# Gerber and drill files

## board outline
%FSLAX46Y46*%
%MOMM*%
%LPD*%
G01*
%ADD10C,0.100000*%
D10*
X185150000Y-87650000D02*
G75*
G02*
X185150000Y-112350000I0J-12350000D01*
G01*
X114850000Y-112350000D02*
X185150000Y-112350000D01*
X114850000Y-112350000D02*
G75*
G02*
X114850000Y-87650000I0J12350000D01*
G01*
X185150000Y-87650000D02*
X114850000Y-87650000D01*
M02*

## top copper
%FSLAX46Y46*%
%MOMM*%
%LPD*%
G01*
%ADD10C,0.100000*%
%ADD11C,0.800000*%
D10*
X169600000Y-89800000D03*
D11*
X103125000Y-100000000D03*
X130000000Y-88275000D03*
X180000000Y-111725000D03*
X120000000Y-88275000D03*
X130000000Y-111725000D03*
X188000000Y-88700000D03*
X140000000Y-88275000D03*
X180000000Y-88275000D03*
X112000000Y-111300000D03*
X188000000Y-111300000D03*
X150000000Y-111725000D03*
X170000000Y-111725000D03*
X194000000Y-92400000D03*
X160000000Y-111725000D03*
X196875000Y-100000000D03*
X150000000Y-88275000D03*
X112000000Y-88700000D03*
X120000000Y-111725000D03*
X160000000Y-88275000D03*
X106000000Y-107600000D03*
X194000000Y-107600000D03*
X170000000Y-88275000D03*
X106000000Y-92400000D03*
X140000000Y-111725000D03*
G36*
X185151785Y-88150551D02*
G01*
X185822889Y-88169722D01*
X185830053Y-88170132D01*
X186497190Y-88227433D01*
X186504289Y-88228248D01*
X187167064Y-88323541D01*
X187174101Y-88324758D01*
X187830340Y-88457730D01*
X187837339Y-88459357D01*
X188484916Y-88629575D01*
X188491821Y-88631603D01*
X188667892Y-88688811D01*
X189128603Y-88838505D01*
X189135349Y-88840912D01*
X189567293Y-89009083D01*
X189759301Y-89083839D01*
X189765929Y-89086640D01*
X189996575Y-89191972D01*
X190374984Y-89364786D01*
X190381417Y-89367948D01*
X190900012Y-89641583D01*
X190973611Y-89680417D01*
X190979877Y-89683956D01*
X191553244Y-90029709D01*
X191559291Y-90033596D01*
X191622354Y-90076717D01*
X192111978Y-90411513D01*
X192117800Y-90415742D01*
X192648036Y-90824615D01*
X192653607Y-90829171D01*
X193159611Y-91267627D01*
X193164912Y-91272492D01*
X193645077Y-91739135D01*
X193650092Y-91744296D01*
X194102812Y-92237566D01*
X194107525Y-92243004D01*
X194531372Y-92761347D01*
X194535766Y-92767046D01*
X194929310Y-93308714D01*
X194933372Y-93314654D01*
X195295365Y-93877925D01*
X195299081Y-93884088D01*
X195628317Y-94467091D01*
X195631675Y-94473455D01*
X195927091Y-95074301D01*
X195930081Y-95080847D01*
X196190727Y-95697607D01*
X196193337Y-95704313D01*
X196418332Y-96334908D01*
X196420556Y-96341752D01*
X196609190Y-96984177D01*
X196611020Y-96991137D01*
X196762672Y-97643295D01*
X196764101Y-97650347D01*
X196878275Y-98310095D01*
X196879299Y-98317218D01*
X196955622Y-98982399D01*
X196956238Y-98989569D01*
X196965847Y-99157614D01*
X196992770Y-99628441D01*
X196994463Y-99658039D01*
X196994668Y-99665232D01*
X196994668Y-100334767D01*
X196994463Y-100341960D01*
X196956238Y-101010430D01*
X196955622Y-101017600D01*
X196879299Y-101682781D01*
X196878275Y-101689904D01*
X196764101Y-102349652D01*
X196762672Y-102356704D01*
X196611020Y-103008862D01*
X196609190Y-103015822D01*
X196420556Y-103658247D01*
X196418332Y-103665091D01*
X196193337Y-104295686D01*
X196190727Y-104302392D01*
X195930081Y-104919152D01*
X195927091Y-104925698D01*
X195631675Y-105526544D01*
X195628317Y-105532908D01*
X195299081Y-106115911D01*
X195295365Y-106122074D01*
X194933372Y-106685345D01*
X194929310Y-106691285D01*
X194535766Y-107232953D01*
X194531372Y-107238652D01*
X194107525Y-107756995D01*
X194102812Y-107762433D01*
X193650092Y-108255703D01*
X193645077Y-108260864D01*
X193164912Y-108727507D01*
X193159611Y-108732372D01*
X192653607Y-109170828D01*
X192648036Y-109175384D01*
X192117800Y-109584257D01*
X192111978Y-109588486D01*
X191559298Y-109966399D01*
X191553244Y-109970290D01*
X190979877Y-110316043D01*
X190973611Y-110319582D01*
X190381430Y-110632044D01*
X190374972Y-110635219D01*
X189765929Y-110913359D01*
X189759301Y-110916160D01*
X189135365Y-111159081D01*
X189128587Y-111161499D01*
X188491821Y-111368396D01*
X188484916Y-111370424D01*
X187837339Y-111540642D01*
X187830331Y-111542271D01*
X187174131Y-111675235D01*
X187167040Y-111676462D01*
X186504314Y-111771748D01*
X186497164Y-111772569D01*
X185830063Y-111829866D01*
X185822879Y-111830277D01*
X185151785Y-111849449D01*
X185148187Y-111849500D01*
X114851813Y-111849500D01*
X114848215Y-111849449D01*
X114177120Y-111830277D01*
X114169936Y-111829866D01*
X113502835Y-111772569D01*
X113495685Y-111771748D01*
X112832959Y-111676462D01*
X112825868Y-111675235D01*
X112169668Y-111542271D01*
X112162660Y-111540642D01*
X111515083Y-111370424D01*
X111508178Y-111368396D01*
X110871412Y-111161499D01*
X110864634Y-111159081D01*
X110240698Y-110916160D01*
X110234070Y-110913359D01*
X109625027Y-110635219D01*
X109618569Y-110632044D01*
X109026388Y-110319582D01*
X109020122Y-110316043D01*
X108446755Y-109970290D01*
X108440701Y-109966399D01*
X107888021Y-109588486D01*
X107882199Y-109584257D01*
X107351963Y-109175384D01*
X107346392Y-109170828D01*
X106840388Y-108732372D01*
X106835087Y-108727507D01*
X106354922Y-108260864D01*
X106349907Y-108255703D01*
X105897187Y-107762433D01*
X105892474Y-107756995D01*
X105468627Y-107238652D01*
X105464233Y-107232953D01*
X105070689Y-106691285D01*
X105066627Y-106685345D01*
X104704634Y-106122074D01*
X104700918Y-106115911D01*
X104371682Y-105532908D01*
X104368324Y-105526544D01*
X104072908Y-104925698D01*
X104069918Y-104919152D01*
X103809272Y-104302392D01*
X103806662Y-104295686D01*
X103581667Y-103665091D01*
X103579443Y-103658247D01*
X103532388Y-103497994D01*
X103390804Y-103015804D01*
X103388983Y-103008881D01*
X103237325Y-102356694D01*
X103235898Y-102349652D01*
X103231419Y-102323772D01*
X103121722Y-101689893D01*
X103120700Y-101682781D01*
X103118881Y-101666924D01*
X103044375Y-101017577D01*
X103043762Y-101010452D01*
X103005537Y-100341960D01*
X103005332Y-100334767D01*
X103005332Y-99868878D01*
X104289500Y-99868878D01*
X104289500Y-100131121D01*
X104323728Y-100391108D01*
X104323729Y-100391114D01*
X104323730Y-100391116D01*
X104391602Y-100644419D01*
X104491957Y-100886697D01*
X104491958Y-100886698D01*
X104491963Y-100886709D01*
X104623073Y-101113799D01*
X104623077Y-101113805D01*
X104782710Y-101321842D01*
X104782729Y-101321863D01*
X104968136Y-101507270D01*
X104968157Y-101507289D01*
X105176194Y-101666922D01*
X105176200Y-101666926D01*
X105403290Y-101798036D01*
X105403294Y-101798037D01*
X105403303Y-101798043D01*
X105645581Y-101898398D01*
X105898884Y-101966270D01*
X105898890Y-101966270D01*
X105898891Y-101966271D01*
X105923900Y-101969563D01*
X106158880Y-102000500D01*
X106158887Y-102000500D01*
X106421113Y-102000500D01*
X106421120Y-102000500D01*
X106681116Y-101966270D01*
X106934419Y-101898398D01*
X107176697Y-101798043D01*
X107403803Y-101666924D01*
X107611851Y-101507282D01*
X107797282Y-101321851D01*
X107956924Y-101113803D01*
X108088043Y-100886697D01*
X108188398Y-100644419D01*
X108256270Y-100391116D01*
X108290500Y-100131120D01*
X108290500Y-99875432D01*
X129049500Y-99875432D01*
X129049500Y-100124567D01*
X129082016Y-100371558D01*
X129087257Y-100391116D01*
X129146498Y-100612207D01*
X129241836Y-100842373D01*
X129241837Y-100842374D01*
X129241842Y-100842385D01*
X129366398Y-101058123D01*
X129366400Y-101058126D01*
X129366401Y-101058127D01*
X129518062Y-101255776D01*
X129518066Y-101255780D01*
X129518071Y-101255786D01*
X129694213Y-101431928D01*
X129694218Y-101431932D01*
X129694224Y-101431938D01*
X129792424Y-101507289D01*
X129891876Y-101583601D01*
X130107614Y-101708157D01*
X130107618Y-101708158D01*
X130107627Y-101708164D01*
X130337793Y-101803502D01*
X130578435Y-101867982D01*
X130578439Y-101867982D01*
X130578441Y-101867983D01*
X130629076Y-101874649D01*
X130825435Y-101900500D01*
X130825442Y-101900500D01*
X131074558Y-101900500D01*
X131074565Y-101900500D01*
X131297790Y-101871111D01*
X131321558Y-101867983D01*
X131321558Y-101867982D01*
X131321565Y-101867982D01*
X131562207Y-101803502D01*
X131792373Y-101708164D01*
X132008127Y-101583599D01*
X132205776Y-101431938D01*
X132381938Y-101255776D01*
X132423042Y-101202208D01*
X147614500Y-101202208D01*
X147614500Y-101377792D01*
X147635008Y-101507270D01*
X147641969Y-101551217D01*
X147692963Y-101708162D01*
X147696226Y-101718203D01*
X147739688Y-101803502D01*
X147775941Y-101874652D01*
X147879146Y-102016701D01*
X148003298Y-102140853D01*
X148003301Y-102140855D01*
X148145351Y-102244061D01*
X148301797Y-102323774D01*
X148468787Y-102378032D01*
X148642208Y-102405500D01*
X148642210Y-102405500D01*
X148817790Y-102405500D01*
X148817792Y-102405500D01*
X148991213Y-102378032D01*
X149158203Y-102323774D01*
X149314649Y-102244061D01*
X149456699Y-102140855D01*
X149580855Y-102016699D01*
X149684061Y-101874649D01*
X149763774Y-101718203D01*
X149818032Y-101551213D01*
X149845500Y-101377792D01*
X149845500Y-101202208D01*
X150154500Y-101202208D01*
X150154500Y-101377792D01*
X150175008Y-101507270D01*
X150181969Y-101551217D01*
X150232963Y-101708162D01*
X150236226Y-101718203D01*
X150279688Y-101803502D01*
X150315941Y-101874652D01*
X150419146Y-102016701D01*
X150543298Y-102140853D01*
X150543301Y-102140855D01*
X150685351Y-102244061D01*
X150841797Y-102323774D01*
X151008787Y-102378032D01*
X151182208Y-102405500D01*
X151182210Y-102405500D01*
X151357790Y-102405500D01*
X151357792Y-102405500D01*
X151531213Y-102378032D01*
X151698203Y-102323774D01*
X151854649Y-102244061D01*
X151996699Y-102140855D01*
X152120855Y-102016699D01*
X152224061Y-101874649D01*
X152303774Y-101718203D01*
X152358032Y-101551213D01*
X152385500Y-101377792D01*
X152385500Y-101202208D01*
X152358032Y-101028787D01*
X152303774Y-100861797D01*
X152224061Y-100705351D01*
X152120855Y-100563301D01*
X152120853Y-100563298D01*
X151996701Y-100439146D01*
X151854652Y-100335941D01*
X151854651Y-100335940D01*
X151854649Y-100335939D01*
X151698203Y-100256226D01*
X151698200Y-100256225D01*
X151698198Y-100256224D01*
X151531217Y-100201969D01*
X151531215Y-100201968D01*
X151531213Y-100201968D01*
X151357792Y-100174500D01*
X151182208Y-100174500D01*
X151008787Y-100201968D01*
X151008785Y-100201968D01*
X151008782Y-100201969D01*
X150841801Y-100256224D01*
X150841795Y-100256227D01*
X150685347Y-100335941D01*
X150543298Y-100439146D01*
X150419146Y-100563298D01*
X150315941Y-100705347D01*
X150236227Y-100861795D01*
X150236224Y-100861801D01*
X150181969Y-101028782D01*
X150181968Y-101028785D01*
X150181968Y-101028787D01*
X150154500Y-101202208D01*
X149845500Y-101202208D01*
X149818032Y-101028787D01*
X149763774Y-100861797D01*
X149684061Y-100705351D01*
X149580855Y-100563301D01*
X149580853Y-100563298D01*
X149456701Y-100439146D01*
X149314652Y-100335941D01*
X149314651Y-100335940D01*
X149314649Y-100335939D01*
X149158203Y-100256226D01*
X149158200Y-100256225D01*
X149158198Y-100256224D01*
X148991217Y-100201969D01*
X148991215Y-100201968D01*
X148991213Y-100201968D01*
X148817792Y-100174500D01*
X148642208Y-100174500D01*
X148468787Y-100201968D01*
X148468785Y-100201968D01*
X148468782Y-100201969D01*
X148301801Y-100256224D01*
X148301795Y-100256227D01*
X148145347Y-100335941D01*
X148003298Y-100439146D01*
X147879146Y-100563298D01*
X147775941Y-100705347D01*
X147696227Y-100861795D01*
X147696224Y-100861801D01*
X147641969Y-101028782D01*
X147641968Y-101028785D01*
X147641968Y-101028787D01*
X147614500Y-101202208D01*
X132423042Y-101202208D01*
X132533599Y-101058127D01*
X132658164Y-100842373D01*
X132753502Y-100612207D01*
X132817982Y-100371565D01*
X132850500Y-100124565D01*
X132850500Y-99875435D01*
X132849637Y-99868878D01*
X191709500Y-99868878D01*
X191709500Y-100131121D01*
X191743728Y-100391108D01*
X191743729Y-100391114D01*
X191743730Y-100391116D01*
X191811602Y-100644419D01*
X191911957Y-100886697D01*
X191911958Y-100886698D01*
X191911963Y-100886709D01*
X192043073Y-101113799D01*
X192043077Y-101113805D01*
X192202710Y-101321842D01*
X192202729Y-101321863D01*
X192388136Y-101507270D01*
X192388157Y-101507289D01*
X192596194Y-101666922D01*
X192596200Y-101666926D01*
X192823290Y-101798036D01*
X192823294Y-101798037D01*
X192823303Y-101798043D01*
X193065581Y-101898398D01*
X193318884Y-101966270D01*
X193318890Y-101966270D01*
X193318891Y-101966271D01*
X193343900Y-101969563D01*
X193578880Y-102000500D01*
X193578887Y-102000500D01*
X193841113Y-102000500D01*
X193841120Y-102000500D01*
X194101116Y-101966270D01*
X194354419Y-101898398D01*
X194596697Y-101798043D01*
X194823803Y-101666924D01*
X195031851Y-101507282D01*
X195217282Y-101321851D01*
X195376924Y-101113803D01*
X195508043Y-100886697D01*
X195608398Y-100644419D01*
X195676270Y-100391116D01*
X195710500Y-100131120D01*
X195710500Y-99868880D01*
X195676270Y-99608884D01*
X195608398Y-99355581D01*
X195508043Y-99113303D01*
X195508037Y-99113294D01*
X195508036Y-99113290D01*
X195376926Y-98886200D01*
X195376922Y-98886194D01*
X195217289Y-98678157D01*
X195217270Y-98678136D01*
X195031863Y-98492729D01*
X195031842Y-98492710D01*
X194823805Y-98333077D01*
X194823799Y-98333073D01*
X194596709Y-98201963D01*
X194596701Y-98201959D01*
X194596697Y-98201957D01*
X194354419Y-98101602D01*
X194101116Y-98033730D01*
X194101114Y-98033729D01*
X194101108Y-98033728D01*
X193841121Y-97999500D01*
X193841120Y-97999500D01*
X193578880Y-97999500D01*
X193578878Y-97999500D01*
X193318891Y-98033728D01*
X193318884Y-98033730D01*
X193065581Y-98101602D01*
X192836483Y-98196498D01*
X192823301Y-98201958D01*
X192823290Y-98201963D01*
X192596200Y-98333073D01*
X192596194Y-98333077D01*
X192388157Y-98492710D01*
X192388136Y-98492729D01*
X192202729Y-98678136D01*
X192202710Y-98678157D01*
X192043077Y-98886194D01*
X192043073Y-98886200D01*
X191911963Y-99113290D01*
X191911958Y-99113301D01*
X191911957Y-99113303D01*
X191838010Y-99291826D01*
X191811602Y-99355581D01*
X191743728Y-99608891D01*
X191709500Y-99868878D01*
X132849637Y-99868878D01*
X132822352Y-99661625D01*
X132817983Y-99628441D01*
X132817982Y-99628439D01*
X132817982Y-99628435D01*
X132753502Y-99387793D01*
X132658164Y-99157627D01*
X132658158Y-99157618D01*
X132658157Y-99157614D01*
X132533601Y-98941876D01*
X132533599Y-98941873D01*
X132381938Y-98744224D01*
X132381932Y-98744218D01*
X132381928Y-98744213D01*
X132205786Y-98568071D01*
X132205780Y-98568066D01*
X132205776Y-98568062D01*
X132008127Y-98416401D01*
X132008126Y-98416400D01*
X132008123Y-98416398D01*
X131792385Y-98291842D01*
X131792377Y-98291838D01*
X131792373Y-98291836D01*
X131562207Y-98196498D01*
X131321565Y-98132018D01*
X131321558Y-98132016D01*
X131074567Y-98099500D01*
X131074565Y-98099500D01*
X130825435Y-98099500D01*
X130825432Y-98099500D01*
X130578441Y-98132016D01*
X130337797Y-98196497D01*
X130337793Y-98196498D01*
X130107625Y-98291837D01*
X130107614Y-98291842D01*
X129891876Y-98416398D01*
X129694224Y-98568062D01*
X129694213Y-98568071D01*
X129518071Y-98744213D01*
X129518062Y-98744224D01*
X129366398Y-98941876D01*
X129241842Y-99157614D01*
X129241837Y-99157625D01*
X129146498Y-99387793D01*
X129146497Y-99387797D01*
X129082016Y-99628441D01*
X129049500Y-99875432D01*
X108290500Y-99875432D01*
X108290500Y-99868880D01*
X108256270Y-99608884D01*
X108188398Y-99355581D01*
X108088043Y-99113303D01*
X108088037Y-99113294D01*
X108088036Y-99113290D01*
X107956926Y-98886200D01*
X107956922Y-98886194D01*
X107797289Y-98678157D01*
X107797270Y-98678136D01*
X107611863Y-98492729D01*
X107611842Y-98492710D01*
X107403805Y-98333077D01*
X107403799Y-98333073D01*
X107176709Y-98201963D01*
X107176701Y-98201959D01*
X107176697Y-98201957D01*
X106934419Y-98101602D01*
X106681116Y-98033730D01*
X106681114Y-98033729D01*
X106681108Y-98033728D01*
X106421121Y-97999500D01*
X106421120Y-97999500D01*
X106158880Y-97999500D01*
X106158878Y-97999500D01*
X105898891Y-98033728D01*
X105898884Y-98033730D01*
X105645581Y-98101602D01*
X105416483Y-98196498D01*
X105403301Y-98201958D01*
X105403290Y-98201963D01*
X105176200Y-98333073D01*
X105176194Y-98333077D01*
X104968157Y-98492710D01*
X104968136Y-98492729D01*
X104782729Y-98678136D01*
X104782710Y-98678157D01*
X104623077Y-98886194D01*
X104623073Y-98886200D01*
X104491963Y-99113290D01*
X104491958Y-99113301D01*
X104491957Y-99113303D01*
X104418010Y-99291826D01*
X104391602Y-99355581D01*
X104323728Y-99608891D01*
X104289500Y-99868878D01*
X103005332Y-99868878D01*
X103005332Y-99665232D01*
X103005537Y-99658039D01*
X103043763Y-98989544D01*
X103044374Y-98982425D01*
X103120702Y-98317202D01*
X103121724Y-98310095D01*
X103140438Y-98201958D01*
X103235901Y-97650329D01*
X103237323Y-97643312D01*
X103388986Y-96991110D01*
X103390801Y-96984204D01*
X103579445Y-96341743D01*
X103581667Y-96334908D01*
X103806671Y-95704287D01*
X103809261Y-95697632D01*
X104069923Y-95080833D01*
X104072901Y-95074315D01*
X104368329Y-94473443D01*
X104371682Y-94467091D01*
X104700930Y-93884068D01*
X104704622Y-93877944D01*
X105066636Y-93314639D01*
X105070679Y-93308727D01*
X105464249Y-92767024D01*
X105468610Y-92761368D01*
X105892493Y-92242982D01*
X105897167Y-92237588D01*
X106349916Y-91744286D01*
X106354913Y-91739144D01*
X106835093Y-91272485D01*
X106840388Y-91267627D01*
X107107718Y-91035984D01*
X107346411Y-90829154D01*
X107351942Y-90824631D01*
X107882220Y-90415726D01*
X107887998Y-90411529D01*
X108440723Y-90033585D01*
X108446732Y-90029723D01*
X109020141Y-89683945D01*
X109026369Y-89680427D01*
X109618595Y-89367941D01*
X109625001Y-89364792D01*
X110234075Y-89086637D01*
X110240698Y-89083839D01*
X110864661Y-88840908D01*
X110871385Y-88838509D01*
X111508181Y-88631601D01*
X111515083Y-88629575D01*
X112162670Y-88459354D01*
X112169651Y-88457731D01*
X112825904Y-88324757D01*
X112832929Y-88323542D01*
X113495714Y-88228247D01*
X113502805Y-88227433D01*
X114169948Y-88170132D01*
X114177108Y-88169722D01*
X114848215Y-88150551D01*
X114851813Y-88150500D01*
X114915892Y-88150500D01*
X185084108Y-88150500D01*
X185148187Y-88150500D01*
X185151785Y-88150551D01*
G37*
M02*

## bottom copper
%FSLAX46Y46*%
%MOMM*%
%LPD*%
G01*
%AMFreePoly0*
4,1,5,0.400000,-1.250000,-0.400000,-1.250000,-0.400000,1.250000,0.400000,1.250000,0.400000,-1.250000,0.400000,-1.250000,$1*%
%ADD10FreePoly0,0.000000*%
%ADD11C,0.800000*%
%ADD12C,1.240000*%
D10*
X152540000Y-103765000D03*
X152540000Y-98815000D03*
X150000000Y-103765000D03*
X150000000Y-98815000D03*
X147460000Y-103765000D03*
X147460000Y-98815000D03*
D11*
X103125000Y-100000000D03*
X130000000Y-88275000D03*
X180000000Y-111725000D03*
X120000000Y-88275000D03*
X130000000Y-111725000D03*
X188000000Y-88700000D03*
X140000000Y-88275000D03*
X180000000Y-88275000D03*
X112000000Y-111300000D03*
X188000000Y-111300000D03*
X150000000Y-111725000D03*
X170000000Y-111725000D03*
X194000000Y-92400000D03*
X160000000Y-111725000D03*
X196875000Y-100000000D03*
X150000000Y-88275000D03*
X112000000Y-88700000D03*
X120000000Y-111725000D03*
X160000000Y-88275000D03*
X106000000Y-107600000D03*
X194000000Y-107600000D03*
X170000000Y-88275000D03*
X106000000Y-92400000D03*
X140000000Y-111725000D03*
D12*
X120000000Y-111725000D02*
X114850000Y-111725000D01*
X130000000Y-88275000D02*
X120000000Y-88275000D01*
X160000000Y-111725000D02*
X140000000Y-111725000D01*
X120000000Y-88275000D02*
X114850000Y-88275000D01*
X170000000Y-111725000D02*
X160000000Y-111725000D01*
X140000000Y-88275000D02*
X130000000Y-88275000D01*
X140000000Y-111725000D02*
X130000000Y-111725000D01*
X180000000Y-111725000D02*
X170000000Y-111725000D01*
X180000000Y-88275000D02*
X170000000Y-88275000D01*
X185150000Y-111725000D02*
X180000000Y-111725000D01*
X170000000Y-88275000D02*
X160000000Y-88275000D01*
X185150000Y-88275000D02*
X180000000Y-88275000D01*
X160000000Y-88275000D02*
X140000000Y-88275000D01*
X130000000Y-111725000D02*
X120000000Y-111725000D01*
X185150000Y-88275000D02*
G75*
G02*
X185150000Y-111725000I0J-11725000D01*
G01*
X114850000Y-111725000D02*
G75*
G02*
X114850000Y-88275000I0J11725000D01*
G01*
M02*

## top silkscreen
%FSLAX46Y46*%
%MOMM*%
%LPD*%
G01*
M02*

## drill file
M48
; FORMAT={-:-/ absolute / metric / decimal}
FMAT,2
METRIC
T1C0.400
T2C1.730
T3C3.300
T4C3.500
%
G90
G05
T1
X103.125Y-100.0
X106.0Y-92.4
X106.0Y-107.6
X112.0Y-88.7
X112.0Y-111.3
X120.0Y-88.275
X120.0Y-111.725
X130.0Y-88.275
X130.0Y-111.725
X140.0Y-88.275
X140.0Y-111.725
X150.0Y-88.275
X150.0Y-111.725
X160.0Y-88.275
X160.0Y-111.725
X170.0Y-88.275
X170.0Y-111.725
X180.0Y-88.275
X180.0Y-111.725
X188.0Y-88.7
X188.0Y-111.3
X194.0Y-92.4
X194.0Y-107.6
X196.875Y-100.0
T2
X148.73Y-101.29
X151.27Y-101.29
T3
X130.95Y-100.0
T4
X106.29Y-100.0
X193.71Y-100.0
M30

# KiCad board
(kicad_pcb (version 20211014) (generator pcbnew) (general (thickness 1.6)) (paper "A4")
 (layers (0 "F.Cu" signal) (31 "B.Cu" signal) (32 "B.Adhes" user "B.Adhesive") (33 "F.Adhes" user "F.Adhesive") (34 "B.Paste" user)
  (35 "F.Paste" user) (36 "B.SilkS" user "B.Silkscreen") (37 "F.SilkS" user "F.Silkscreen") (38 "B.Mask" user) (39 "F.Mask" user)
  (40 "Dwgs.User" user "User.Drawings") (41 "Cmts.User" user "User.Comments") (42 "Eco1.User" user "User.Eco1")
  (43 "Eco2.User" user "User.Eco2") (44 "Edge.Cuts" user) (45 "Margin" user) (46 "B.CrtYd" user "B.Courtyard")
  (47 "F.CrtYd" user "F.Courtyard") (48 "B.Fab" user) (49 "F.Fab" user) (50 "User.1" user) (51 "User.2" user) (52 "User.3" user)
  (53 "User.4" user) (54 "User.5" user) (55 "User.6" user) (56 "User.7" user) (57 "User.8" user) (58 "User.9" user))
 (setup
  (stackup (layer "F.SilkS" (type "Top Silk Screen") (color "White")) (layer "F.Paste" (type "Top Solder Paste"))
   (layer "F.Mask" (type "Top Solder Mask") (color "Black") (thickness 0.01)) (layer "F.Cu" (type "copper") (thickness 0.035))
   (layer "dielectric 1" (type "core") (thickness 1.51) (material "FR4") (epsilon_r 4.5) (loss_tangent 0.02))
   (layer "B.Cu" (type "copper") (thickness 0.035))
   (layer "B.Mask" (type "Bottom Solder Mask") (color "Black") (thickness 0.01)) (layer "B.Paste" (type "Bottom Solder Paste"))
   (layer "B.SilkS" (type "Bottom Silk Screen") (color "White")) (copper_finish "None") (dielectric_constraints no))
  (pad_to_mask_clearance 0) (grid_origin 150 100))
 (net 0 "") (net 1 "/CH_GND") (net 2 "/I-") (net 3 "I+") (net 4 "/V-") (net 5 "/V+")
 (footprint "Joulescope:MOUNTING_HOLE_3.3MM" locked (layer "F.Cu") (at 130.95 100)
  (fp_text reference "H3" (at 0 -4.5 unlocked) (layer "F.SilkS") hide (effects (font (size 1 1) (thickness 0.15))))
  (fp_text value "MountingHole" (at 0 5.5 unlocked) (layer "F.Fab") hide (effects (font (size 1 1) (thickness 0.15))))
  (pad "" np_thru_hole circle locked (at 0 0) (size 3.3 3.3) (drill 3.3) (layers *.Mask)))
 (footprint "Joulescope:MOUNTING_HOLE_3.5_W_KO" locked (layer "F.Cu") (at 193.71 100)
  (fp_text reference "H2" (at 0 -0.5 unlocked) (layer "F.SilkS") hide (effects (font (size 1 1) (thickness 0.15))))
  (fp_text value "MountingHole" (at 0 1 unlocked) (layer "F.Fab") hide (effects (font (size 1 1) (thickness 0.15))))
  (pad "" np_thru_hole circle locked (at 0 0) (size 3.5 3.5) (drill 3.5) (layers *.Mask))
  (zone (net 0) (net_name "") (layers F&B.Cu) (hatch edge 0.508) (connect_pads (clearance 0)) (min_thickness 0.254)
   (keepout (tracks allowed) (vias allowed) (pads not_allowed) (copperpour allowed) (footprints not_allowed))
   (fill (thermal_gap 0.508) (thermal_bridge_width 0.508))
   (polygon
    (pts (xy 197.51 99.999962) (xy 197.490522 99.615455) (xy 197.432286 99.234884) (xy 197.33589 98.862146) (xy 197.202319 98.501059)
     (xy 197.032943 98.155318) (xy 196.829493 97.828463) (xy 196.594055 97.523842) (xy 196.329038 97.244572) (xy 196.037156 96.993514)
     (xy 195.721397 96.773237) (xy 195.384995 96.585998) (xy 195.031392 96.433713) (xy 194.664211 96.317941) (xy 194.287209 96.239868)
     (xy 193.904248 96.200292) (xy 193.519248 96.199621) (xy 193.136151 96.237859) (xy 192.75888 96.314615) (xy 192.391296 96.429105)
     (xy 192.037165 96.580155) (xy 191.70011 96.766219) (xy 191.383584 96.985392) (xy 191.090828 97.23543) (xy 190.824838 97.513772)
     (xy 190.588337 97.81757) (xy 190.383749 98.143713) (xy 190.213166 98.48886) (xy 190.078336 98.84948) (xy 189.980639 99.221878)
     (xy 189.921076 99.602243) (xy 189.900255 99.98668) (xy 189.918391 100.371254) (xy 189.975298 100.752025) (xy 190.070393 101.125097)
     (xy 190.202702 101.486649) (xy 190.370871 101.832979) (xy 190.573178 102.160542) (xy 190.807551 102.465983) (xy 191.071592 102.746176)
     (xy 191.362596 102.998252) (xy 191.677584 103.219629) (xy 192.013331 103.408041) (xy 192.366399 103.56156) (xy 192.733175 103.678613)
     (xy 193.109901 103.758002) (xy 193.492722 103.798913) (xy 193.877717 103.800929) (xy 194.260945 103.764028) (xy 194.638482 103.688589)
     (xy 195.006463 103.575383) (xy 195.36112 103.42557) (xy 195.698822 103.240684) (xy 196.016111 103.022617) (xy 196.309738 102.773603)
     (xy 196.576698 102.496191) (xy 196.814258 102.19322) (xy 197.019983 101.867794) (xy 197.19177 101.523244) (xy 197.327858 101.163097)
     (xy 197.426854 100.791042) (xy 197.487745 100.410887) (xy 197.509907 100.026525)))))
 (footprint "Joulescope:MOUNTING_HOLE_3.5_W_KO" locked (layer "F.Cu") (at 106.29 100)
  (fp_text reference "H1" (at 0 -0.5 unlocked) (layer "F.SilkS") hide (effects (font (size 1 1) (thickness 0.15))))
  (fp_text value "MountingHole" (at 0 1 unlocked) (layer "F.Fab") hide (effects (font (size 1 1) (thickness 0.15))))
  (pad "" np_thru_hole circle locked (at 0 0) (size 3.5 3.5) (drill 3.5) (layers *.Mask))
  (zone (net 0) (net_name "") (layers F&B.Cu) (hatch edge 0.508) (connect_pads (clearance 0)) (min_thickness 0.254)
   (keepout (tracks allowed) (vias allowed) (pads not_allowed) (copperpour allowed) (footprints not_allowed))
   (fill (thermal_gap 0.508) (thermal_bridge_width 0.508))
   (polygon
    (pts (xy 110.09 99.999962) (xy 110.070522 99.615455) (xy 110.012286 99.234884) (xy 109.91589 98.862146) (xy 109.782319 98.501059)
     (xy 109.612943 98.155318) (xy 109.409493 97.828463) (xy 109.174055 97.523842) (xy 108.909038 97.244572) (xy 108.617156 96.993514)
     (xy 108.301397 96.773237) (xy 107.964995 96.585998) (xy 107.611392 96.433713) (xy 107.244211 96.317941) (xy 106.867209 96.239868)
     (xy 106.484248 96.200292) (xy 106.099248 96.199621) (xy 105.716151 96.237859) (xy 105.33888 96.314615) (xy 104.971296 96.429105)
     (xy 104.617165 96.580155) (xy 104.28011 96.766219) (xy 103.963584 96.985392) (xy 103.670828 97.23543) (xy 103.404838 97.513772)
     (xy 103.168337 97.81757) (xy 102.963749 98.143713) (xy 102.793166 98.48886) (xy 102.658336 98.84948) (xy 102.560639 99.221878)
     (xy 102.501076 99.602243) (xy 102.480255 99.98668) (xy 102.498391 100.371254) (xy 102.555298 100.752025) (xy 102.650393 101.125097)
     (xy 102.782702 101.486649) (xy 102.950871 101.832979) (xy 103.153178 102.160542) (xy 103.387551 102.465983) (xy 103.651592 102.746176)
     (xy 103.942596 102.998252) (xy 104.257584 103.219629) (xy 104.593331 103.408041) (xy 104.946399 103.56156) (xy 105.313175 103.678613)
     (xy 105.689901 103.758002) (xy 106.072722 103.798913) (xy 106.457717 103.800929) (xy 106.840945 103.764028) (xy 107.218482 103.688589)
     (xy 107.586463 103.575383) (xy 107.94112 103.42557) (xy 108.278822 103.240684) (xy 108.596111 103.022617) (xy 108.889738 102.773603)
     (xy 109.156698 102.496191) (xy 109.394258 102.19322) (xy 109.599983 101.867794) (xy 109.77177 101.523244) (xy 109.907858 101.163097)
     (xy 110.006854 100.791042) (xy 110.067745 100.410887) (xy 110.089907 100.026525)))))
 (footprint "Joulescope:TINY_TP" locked (layer "F.Cu") (at 169.6 89.5)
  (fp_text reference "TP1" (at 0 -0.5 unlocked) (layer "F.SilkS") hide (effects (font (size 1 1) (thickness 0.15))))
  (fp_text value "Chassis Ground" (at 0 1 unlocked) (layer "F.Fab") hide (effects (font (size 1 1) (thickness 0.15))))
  (pad "1" smd circle locked (at 0 0.3) (size 0.1 0.1) (layers "F.Cu" "F.Paste" "F.Mask") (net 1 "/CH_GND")))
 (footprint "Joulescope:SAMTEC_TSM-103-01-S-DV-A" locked (layer "B.Cu") (at 150 101.29)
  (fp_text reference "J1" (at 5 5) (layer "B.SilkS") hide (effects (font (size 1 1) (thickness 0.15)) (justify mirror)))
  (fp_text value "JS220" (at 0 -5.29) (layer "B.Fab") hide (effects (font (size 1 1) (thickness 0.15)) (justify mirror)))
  (pad "" np_thru_hole circle locked (at 1.27 0) (size 1.73 1.73) (drill 1.73) (layers *.Cu *.Mask))
  (pad "" np_thru_hole circle locked (at -1.27 0) (size 1.73 1.73) (drill 1.73) (layers *.Cu *.Mask))
  (pad "1" smd custom locked (at 2.54 2.475) (size 0.8 2.5) (layers "B.Cu") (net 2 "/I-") (zone_connect 0)
   (options (clearance outline) (anchor rect)) (primitives))
  (pad "2" smd custom locked (at 2.54 -2.475) (size 0.8 2.5) (layers "B.Cu") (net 2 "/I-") (zone_connect 0)
   (options (clearance outline) (anchor rect)) (primitives))
  (pad "3" smd custom locked (at 0 2.475) (size 0.8 2.5) (layers "B.Cu") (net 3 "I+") (zone_connect 0)
   (options (clearance outline) (anchor rect)) (primitives))
  (pad "4" smd custom locked (at 0 -2.475) (size 0.8 2.5) (layers "B.Cu") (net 3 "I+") (zone_connect 0)
   (options (clearance outline) (anchor rect)) (primitives))
  (pad "5" smd custom locked (at -2.54 2.475) (size 0.8 2.5) (layers "B.Cu") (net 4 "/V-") (zone_connect 0)
   (options (clearance outline) (anchor rect)) (primitives))
  (pad "6" smd custom locked (at -2.54 -2.475) (size 0.8 2.5) (layers "B.Cu") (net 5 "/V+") (zone_connect 0)
   (options (clearance outline) (anchor rect)) (primitives)))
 (gr_arc locked (start 185.15 87.65) (mid 197.5 100) (end 185.15 112.35) (layer "Edge.Cuts") (width 0.1))
 (gr_line locked (start 114.85 112.35) (end 185.15 112.35) (layer "Edge.Cuts") (width 0.1))
 (gr_arc locked (start 114.85 112.35) (mid 102.5 100) (end 114.85 87.65) (layer "Edge.Cuts") (width 0.1))
 (gr_line locked (start 185.15 87.65) (end 114.85 87.65) (layer "Edge.Cuts") (width 0.1))
 (via locked (at 103.125 100) (size 0.8) (drill 0.4) (layers "F.Cu" "B.Cu") (free) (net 1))
 (via locked (at 130 88.275) (size 0.8) (drill 0.4) (layers "F.Cu" "B.Cu") (free) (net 1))
 (via locked (at 180 111.725) (size 0.8) (drill 0.4) (layers "F.Cu" "B.Cu") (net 1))
 (via locked (at 120 88.275) (size 0.8) (drill 0.4) (layers "F.Cu" "B.Cu") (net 1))
 (via locked (at 130 111.725) (size 0.8) (drill 0.4) (layers "F.Cu" "B.Cu") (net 1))
 (via locked (at 188 88.7) (size 0.8) (drill 0.4) (layers "F.Cu" "B.Cu") (free) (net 1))
 (via locked (at 140 88.275) (size 0.8) (drill 0.4) (layers "F.Cu" "B.Cu") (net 1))
 (via locked (at 180 88.275) (size 0.8) (drill 0.4) (layers "F.Cu" "B.Cu") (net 1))
 (via locked (at 112 111.3) (size 0.8) (drill 0.4) (layers "F.Cu" "B.Cu") (free) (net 1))
 (via locked (at 188 111.3) (size 0.8) (drill 0.4) (layers "F.Cu" "B.Cu") (free) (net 1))
 (via locked (at 150 111.725) (size 0.8) (drill 0.4) (layers "F.Cu" "B.Cu") (free) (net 1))
 (via locked (at 170 111.725) (size 0.8) (drill 0.4) (layers "F.Cu" "B.Cu") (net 1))
 (via locked (at 194 92.4) (size 0.8) (drill 0.4) (layers "F.Cu" "B.Cu") (free) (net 1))
 (via locked (at 160 111.725) (size 0.8) (drill 0.4) (layers "F.Cu" "B.Cu") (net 1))
 (via locked (at 196.875 100) (size 0.8) (drill 0.4) (layers "F.Cu" "B.Cu") (free) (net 1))
 (via locked (at 150 88.275) (size 0.8) (drill 0.4) (layers "F.Cu" "B.Cu") (free) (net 1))
 (via locked (at 112 88.7) (size 0.8) (drill 0.4) (layers "F.Cu" "B.Cu") (free) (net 1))
 (via locked (at 120 111.725) (size 0.8) (drill 0.4) (layers "F.Cu" "B.Cu") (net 1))
 (via locked (at 160 88.275) (size 0.8) (drill 0.4) (layers "F.Cu" "B.Cu") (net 1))
 (via locked (at 106 107.6) (size 0.8) (drill 0.4) (layers "F.Cu" "B.Cu") (free) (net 1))
 (via locked (at 194 107.6) (size 0.8) (drill 0.4) (layers "F.Cu" "B.Cu") (free) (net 1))
 (via locked (at 170 88.275) (size 0.8) (drill 0.4) (layers "F.Cu" "B.Cu") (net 1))
 (via locked (at 106 92.4) (size 0.8) (drill 0.4) (layers "F.Cu" "B.Cu") (free) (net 1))
 (via locked (at 140 111.725) (size 0.8) (drill 0.4) (layers "F.Cu" "B.Cu") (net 1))
 (segment locked (start 120 111.725) (end 114.85 111.725) (width 1.24) (layer "B.Cu") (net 1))
 (segment locked (start 130 88.275) (end 120 88.275) (width 1.24) (layer "B.Cu") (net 1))
 (segment locked (start 160 111.725) (end 140 111.725) (width 1.24) (layer "B.Cu") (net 1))
 (segment locked (start 120 88.275) (end 114.85 88.275) (width 1.24) (layer "B.Cu") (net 1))
 (segment locked (start 170 111.725) (end 160 111.725) (width 1.24) (layer "B.Cu") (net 1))
 (segment locked (start 140 88.275) (end 130 88.275) (width 1.24) (layer "B.Cu") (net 1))
 (segment locked (start 140 111.725) (end 130 111.725) (width 1.24) (layer "B.Cu") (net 1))
 (segment locked (start 180 111.725) (end 170 111.725) (width 1.24) (layer "B.Cu") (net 1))
 (segment locked (start 180 88.275) (end 170 88.275) (width 1.24) (layer "B.Cu") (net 1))
 (segment locked (start 185.15 111.725) (end 180 111.725) (width 1.24) (layer "B.Cu") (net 1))
 (segment locked (start 170 88.275) (end 160 88.275) (width 1.24) (layer "B.Cu") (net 1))
 (segment locked (start 185.15 88.275) (end 180 88.275) (width 1.24) (layer "B.Cu") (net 1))
 (segment locked (start 160 88.275) (end 140 88.275) (width 1.24) (layer "B.Cu") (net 1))
 (segment locked (start 130 111.725) (end 120 111.725) (width 1.24) (layer "B.Cu") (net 1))
 (arc locked (start 185.15 88.275) (mid 196.875 100) (end 185.15 111.725) (width 1.24) (layer "B.Cu") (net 1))
 (arc locked (start 114.85 111.725) (mid 103.125 100) (end 114.85 88.275) (width 1.24) (layer "B.Cu") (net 1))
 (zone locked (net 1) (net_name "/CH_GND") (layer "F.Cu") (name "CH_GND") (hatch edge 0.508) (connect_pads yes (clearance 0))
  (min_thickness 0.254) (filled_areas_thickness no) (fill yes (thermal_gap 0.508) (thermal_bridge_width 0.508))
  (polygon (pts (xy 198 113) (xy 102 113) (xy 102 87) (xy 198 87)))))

